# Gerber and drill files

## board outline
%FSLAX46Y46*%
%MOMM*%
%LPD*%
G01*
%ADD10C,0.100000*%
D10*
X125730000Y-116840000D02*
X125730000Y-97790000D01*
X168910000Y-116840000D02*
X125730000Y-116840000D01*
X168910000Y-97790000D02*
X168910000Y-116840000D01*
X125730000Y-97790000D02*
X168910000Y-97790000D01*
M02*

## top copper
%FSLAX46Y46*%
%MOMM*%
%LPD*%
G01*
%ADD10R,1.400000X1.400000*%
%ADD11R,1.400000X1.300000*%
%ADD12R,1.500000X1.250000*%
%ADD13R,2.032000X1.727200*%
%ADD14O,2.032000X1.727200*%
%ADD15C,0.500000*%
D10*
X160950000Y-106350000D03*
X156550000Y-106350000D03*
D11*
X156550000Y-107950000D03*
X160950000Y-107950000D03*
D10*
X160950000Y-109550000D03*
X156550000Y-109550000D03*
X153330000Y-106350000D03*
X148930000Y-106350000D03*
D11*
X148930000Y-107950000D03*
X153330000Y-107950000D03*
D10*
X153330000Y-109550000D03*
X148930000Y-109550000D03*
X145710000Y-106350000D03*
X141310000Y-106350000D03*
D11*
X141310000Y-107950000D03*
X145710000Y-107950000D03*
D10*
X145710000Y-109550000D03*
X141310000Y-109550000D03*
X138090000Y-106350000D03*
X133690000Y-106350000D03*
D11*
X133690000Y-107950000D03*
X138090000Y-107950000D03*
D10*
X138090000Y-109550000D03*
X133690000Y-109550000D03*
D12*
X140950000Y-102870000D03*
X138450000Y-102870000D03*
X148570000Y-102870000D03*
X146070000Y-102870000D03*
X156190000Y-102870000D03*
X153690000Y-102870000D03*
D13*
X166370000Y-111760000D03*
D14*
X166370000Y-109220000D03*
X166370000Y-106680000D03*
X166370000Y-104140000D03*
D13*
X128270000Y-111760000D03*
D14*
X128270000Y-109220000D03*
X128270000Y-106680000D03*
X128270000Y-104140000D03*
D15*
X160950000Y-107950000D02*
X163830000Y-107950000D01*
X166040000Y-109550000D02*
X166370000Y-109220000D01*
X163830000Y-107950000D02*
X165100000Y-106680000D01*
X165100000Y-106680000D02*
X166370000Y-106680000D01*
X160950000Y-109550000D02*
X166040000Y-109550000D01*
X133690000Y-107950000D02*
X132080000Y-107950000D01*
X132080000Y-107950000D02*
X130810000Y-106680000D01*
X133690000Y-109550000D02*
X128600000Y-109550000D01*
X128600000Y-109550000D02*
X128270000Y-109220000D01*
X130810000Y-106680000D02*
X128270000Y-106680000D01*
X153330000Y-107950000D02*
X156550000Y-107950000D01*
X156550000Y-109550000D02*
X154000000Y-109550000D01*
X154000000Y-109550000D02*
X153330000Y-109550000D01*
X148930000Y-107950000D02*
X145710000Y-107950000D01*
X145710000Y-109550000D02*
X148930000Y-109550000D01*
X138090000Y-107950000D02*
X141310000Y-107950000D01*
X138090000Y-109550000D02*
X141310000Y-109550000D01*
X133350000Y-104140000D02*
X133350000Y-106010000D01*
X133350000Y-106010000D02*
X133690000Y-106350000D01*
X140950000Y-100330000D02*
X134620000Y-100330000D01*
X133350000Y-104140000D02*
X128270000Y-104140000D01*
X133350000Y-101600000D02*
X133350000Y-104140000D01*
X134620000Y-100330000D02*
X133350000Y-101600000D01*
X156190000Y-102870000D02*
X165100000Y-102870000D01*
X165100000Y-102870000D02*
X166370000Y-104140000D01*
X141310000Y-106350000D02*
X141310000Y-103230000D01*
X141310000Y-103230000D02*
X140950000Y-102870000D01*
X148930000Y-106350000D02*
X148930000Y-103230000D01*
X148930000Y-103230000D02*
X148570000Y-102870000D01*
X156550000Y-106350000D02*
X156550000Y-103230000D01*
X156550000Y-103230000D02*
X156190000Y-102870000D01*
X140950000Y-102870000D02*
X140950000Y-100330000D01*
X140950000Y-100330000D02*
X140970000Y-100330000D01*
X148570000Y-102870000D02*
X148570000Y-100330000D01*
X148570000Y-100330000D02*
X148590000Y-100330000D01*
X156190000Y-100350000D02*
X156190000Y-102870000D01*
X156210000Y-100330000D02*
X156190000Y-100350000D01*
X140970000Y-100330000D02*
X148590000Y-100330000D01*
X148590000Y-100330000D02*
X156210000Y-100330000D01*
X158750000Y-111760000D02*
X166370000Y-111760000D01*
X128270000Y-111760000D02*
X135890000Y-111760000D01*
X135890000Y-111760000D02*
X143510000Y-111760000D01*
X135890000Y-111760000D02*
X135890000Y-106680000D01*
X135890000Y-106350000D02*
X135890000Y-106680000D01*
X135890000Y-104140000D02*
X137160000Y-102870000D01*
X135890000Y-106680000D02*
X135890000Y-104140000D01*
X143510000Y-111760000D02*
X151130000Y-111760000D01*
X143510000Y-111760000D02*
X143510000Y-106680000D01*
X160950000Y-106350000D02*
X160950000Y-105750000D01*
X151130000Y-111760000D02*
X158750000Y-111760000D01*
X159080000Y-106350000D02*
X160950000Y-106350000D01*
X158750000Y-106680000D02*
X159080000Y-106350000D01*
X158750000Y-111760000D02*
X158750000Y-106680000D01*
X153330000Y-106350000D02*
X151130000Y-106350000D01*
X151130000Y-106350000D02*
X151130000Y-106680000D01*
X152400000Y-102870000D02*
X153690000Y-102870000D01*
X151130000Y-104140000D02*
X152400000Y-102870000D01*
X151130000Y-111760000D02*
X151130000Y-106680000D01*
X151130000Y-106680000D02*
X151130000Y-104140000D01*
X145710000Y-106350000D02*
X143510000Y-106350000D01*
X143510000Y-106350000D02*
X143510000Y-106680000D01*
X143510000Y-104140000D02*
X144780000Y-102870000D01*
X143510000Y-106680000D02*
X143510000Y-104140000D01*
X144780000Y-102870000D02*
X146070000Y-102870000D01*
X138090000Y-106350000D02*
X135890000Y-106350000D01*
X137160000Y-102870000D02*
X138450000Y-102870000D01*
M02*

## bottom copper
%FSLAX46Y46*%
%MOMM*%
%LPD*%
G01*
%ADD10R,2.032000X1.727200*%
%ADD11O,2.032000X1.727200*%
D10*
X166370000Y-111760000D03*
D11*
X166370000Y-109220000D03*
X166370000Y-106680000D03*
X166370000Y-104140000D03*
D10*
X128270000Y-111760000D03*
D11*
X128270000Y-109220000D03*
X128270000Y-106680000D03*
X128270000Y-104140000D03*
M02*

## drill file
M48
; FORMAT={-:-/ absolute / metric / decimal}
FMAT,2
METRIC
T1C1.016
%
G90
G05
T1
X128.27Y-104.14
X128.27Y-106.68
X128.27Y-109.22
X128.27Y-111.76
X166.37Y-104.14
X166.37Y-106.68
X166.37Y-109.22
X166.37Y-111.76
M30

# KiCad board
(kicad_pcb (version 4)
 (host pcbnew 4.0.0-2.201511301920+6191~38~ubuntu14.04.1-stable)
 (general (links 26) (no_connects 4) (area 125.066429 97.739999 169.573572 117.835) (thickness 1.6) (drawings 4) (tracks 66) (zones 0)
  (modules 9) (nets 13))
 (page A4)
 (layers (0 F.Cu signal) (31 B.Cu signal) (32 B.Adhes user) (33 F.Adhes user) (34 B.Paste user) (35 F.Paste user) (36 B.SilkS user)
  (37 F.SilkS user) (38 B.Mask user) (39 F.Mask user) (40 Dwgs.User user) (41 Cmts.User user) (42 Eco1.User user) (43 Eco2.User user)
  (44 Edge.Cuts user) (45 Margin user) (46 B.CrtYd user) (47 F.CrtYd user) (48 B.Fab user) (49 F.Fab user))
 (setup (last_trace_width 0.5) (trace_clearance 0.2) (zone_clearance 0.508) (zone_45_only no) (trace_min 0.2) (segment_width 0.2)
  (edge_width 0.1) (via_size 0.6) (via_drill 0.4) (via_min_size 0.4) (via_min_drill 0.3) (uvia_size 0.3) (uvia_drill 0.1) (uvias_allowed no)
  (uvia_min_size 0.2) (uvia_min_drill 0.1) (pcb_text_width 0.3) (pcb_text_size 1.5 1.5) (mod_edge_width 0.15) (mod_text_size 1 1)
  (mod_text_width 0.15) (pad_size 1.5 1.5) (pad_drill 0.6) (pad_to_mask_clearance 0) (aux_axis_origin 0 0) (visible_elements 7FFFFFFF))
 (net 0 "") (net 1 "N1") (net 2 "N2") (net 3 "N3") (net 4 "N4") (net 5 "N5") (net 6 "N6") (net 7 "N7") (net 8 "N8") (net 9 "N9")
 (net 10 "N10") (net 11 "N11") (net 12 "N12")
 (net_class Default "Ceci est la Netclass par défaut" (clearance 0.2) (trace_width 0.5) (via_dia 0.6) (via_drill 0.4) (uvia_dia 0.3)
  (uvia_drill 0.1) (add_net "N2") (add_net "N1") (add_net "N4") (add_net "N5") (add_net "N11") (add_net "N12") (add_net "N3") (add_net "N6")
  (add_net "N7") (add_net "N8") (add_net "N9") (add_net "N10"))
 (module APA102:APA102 (layer F.Cu) (at 158.75 107.95 90)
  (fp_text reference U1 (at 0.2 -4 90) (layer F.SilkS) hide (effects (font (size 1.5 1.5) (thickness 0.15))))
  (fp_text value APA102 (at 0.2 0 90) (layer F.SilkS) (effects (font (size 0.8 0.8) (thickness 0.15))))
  (pad 3 smd rect (at 1.6 2.2 180) (size 1.4 1.4) (layers F.Cu F.Paste F.Mask) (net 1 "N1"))
  (pad 4 smd rect (at 1.6 -2.2 180) (size 1.4 1.4) (layers F.Cu F.Paste F.Mask) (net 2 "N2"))
  (pad 5 smd rect (at 0 -2.2 180) (size 1.4 1.3) (layers F.Cu F.Paste F.Mask) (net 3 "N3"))
  (pad 2 smd rect (at 0 2.2 180) (size 1.4 1.3) (layers F.Cu F.Paste F.Mask) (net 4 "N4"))
  (pad 1 smd rect (at -1.6 2.2 180) (size 1.4 1.4) (layers F.Cu F.Paste F.Mask) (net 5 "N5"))
  (pad 6 smd rect (at -1.6 -2.2 180) (size 1.4 1.4) (layers F.Cu F.Paste F.Mask) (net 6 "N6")))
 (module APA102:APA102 (layer F.Cu) (at 151.13 107.95 90)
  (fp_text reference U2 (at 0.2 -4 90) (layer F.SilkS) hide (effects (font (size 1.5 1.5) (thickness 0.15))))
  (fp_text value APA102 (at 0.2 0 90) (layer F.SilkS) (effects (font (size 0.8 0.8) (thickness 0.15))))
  (pad 3 smd rect (at 1.6 2.2 180) (size 1.4 1.4) (layers F.Cu F.Paste F.Mask) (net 1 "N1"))
  (pad 4 smd rect (at 1.6 -2.2 180) (size 1.4 1.4) (layers F.Cu F.Paste F.Mask) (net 2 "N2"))
  (pad 5 smd rect (at 0 -2.2 180) (size 1.4 1.3) (layers F.Cu F.Paste F.Mask) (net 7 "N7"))
  (pad 2 smd rect (at 0 2.2 180) (size 1.4 1.3) (layers F.Cu F.Paste F.Mask) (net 3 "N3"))
  (pad 1 smd rect (at -1.6 2.2 180) (size 1.4 1.4) (layers F.Cu F.Paste F.Mask) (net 6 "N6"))
  (pad 6 smd rect (at -1.6 -2.2 180) (size 1.4 1.4) (layers F.Cu F.Paste F.Mask) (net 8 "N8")))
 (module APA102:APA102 (layer F.Cu) (at 143.51 107.95 90)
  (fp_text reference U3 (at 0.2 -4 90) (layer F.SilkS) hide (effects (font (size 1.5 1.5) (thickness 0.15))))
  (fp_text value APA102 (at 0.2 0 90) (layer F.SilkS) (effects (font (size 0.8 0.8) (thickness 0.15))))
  (pad 3 smd rect (at 1.6 2.2 180) (size 1.4 1.4) (layers F.Cu F.Paste F.Mask) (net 1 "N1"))
  (pad 4 smd rect (at 1.6 -2.2 180) (size 1.4 1.4) (layers F.Cu F.Paste F.Mask) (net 2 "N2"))
  (pad 5 smd rect (at 0 -2.2 180) (size 1.4 1.3) (layers F.Cu F.Paste F.Mask) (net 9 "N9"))
  (pad 2 smd rect (at 0 2.2 180) (size 1.4 1.3) (layers F.Cu F.Paste F.Mask) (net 7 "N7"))
  (pad 1 smd rect (at -1.6 2.2 180) (size 1.4 1.4) (layers F.Cu F.Paste F.Mask) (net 8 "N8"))
  (pad 6 smd rect (at -1.6 -2.2 180) (size 1.4 1.4) (layers F.Cu F.Paste F.Mask) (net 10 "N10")))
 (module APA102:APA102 (layer F.Cu) (at 135.89 107.95 90)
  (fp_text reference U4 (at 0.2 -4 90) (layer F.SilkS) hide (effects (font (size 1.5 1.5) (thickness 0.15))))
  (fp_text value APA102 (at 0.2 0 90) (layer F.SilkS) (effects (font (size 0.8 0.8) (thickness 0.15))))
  (pad 3 smd rect (at 1.6 2.2 180) (size 1.4 1.4) (layers F.Cu F.Paste F.Mask) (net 1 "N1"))
  (pad 4 smd rect (at 1.6 -2.2 180) (size 1.4 1.4) (layers F.Cu F.Paste F.Mask) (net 2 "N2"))
  (pad 5 smd rect (at 0 -2.2 180) (size 1.4 1.3) (layers F.Cu F.Paste F.Mask) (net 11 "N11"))
  (pad 2 smd rect (at 0 2.2 180) (size 1.4 1.3) (layers F.Cu F.Paste F.Mask) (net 9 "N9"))
  (pad 1 smd rect (at -1.6 2.2 180) (size 1.4 1.4) (layers F.Cu F.Paste F.Mask) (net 10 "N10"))
  (pad 6 smd rect (at -1.6 -2.2 180) (size 1.4 1.4) (layers F.Cu F.Paste F.Mask) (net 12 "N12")))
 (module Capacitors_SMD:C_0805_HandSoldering (layer F.Cu) (at 139.7 102.87 180)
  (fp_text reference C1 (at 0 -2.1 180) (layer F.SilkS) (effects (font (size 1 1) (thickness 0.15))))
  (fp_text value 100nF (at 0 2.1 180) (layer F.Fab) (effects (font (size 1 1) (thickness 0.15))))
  (pad 1 smd rect (at -1.25 0 180) (size 1.5 1.25) (layers F.Cu F.Paste F.Mask) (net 2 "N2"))
  (pad 2 smd rect (at 1.25 0 180) (size 1.5 1.25) (layers F.Cu F.Paste F.Mask) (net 1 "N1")))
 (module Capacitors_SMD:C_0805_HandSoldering (layer F.Cu) (at 147.32 102.87 180)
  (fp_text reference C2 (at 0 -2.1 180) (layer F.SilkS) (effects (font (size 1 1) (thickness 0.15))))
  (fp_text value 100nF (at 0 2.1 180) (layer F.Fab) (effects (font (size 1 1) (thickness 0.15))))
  (pad 1 smd rect (at -1.25 0 180) (size 1.5 1.25) (layers F.Cu F.Paste F.Mask) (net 2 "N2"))
  (pad 2 smd rect (at 1.25 0 180) (size 1.5 1.25) (layers F.Cu F.Paste F.Mask) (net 1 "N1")))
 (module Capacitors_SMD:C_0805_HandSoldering (layer F.Cu) (at 154.94 102.87 180)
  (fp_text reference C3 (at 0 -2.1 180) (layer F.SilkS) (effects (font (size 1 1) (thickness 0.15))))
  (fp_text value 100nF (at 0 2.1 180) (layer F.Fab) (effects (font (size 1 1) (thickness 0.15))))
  (pad 1 smd rect (at -1.25 0 180) (size 1.5 1.25) (layers F.Cu F.Paste F.Mask) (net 2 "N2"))
  (pad 2 smd rect (at 1.25 0 180) (size 1.5 1.25) (layers F.Cu F.Paste F.Mask) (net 1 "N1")))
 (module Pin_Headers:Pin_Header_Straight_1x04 (layer F.Cu) (at 166.37 111.76 180)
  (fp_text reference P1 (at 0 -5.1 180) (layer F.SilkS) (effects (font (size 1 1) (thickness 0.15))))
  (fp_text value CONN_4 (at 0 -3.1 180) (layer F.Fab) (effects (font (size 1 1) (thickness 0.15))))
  (pad 1 thru_hole rect (at 0 0 180) (size 2.032 1.7272) (drill 1.016) (layers *.Cu *.Mask F.SilkS) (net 1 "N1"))
  (pad 2 thru_hole oval (at 0 2.54 180) (size 2.032 1.7272) (drill 1.016) (layers *.Cu *.Mask F.SilkS) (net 4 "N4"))
  (pad 3 thru_hole oval (at 0 5.08 180) (size 2.032 1.7272) (drill 1.016) (layers *.Cu *.Mask F.SilkS) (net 5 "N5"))
  (pad 4 thru_hole oval (at 0 7.62 180) (size 2.032 1.7272) (drill 1.016) (layers *.Cu *.Mask F.SilkS) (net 2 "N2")))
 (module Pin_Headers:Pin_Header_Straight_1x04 (layer F.Cu) (at 128.27 111.76 180)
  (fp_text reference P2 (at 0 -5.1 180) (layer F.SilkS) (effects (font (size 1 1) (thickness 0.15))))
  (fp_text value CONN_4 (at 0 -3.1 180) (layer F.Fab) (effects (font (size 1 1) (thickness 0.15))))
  (pad 1 thru_hole rect (at 0 0 180) (size 2.032 1.7272) (drill 1.016) (layers *.Cu *.Mask F.SilkS) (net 1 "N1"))
  (pad 2 thru_hole oval (at 0 2.54 180) (size 2.032 1.7272) (drill 1.016) (layers *.Cu *.Mask F.SilkS) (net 11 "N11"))
  (pad 3 thru_hole oval (at 0 5.08 180) (size 2.032 1.7272) (drill 1.016) (layers *.Cu *.Mask F.SilkS) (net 12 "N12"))
  (pad 4 thru_hole oval (at 0 7.62 180) (size 2.032 1.7272) (drill 1.016) (layers *.Cu *.Mask F.SilkS) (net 2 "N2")))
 (gr_line (start 125.73 116.84) (end 125.73 97.79) (angle 90) (layer Edge.Cuts) (width 0.1))
 (gr_line (start 168.91 116.84) (end 125.73 116.84) (angle 90) (layer Edge.Cuts) (width 0.1))
 (gr_line (start 168.91 97.79) (end 168.91 116.84) (angle 90) (layer Edge.Cuts) (width 0.1))
 (gr_line (start 125.73 97.79) (end 168.91 97.79) (angle 90) (layer Edge.Cuts) (width 0.1))
 (segment (start 160.95 107.95) (end 163.83 107.95) (width 0.5) (layer F.Cu) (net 4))
 (segment (start 166.04 109.55) (end 166.37 109.22) (width 0.5) (layer F.Cu) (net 4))
 (segment (start 163.83 107.95) (end 165.1 106.68) (width 0.5) (layer F.Cu) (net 4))
 (segment (start 165.1 106.68) (end 166.37 106.68) (width 0.5) (layer F.Cu) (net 5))
 (segment (start 160.95 109.55) (end 166.04 109.55) (width 0.5) (layer F.Cu) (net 5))
 (segment (start 133.69 107.95) (end 132.08 107.95) (width 0.5) (layer F.Cu) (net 11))
 (segment (start 132.08 107.95) (end 130.81 106.68) (width 0.5) (layer F.Cu) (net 11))
 (segment (start 133.69 109.55) (end 128.6 109.55) (width 0.5) (layer F.Cu) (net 11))
 (segment (start 128.6 109.55) (end 128.27 109.22) (width 0.5) (layer F.Cu) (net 11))
 (segment (start 130.81 106.68) (end 128.27 106.68) (width 0.5) (layer F.Cu) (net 12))
 (segment (start 153.33 107.95) (end 156.55 107.95) (width 0.5) (layer F.Cu) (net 3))
 (segment (start 156.55 109.55) (end 154 109.55) (width 0.5) (layer F.Cu) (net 6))
 (segment (start 154 109.55) (end 153.33 109.55) (width 0.5) (layer F.Cu) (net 6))
 (segment (start 148.93 107.95) (end 145.71 107.95) (width 0.5) (layer F.Cu) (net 7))
 (segment (start 145.71 109.55) (end 148.93 109.55) (width 0.5) (layer F.Cu) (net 8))
 (segment (start 138.09 107.95) (end 141.31 107.95) (width 0.5) (layer F.Cu) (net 9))
 (segment (start 138.09 109.55) (end 141.31 109.55) (width 0.5) (layer F.Cu) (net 10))
 (segment (start 133.35 104.14) (end 133.35 106.01) (width 0.5) (layer F.Cu) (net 2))
 (segment (start 133.35 106.01) (end 133.69 106.35) (width 0.5) (layer F.Cu) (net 2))
 (segment (start 140.95 100.33) (end 134.62 100.33) (width 0.5) (layer F.Cu) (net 2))
 (segment (start 133.35 104.14) (end 128.27 104.14) (width 0.5) (layer F.Cu) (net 2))
 (segment (start 133.35 101.6) (end 133.35 104.14) (width 0.5) (layer F.Cu) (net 2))
 (segment (start 134.62 100.33) (end 133.35 101.6) (width 0.5) (layer F.Cu) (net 2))
 (segment (start 156.19 102.87) (end 165.1 102.87) (width 0.5) (layer F.Cu) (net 2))
 (segment (start 165.1 102.87) (end 166.37 104.14) (width 0.5) (layer F.Cu) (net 2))
 (segment (start 141.31 106.35) (end 141.31 103.23) (width 0.5) (layer F.Cu) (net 2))
 (segment (start 141.31 103.23) (end 140.95 102.87) (width 0.5) (layer F.Cu) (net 2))
 (segment (start 148.93 106.35) (end 148.93 103.23) (width 0.5) (layer F.Cu) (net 2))
 (segment (start 148.93 103.23) (end 148.57 102.87) (width 0.5) (layer F.Cu) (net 2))
 (segment (start 156.55 106.35) (end 156.55 103.23) (width 0.5) (layer F.Cu) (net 2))
 (segment (start 156.55 103.23) (end 156.19 102.87) (width 0.5) (layer F.Cu) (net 2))
 (segment (start 140.95 102.87) (end 140.95 100.33) (width 0.5) (layer F.Cu) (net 2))
 (segment (start 140.95 100.33) (end 140.97 100.33) (width 0.5) (layer F.Cu) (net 2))
 (segment (start 148.57 102.87) (end 148.57 100.33) (width 0.5) (layer F.Cu) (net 2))
 (segment (start 148.57 100.33) (end 148.59 100.33) (width 0.5) (layer F.Cu) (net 2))
 (segment (start 156.19 100.35) (end 156.19 102.87) (width 0.5) (layer F.Cu) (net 2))
 (segment (start 156.21 100.33) (end 156.19 100.35) (width 0.5) (layer F.Cu) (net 2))
 (segment (start 140.97 100.33) (end 148.59 100.33) (width 0.5) (layer F.Cu) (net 2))
 (segment (start 148.59 100.33) (end 156.21 100.33) (width 0.5) (layer F.Cu) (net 2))
 (segment (start 158.75 111.76) (end 166.37 111.76) (width 0.5) (layer F.Cu) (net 1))
 (segment (start 128.27 111.76) (end 135.89 111.76) (width 0.5) (layer F.Cu) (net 1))
 (segment (start 135.89 111.76) (end 143.51 111.76) (width 0.5) (layer F.Cu) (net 1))
 (segment (start 135.89 111.76) (end 135.89 106.68) (width 0.5) (layer F.Cu) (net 1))
 (segment (start 135.89 106.35) (end 135.89 106.68) (width 0.5) (layer F.Cu) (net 1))
 (segment (start 135.89 104.14) (end 137.16 102.87) (width 0.5) (layer F.Cu) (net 1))
 (segment (start 135.89 106.68) (end 135.89 104.14) (width 0.5) (layer F.Cu) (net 1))
 (segment (start 143.51 111.76) (end 151.13 111.76) (width 0.5) (layer F.Cu) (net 1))
 (segment (start 143.51 111.76) (end 143.51 106.68) (width 0.5) (layer F.Cu) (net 1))
 (segment (start 160.95 106.35) (end 160.95 105.75) (width 0.5) (layer F.Cu) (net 1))
 (segment (start 151.13 111.76) (end 158.75 111.76) (width 0.5) (layer F.Cu) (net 1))
 (segment (start 159.08 106.35) (end 160.95 106.35) (width 0.5) (layer F.Cu) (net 1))
 (segment (start 158.75 106.68) (end 159.08 106.35) (width 0.5) (layer F.Cu) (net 1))
 (segment (start 158.75 111.76) (end 158.75 106.68) (width 0.5) (layer F.Cu) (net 1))
 (segment (start 153.33 106.35) (end 151.13 106.35) (width 0.5) (layer F.Cu) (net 1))
 (segment (start 151.13 106.35) (end 151.13 106.68) (width 0.5) (layer F.Cu) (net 1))
 (segment (start 152.4 102.87) (end 153.69 102.87) (width 0.5) (layer F.Cu) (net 1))
 (segment (start 151.13 104.14) (end 152.4 102.87) (width 0.5) (layer F.Cu) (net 1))
 (segment (start 151.13 111.76) (end 151.13 106.68) (width 0.5) (layer F.Cu) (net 1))
 (segment (start 151.13 106.68) (end 151.13 104.14) (width 0.5) (layer F.Cu) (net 1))
 (segment (start 145.71 106.35) (end 143.51 106.35) (width 0.5) (layer F.Cu) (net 1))
 (segment (start 143.51 106.35) (end 143.51 106.68) (width 0.5) (layer F.Cu) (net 1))
 (segment (start 143.51 104.14) (end 144.78 102.87) (width 0.5) (layer F.Cu) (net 1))
 (segment (start 143.51 106.68) (end 143.51 104.14) (width 0.5) (layer F.Cu) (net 1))
 (segment (start 144.78 102.87) (end 146.07 102.87) (width 0.5) (layer F.Cu) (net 1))
 (segment (start 138.09 106.35) (end 135.89 106.35) (width 0.5) (layer F.Cu) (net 1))
 (segment (start 137.16 102.87) (end 138.45 102.87) (width 0.5) (layer F.Cu) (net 1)))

